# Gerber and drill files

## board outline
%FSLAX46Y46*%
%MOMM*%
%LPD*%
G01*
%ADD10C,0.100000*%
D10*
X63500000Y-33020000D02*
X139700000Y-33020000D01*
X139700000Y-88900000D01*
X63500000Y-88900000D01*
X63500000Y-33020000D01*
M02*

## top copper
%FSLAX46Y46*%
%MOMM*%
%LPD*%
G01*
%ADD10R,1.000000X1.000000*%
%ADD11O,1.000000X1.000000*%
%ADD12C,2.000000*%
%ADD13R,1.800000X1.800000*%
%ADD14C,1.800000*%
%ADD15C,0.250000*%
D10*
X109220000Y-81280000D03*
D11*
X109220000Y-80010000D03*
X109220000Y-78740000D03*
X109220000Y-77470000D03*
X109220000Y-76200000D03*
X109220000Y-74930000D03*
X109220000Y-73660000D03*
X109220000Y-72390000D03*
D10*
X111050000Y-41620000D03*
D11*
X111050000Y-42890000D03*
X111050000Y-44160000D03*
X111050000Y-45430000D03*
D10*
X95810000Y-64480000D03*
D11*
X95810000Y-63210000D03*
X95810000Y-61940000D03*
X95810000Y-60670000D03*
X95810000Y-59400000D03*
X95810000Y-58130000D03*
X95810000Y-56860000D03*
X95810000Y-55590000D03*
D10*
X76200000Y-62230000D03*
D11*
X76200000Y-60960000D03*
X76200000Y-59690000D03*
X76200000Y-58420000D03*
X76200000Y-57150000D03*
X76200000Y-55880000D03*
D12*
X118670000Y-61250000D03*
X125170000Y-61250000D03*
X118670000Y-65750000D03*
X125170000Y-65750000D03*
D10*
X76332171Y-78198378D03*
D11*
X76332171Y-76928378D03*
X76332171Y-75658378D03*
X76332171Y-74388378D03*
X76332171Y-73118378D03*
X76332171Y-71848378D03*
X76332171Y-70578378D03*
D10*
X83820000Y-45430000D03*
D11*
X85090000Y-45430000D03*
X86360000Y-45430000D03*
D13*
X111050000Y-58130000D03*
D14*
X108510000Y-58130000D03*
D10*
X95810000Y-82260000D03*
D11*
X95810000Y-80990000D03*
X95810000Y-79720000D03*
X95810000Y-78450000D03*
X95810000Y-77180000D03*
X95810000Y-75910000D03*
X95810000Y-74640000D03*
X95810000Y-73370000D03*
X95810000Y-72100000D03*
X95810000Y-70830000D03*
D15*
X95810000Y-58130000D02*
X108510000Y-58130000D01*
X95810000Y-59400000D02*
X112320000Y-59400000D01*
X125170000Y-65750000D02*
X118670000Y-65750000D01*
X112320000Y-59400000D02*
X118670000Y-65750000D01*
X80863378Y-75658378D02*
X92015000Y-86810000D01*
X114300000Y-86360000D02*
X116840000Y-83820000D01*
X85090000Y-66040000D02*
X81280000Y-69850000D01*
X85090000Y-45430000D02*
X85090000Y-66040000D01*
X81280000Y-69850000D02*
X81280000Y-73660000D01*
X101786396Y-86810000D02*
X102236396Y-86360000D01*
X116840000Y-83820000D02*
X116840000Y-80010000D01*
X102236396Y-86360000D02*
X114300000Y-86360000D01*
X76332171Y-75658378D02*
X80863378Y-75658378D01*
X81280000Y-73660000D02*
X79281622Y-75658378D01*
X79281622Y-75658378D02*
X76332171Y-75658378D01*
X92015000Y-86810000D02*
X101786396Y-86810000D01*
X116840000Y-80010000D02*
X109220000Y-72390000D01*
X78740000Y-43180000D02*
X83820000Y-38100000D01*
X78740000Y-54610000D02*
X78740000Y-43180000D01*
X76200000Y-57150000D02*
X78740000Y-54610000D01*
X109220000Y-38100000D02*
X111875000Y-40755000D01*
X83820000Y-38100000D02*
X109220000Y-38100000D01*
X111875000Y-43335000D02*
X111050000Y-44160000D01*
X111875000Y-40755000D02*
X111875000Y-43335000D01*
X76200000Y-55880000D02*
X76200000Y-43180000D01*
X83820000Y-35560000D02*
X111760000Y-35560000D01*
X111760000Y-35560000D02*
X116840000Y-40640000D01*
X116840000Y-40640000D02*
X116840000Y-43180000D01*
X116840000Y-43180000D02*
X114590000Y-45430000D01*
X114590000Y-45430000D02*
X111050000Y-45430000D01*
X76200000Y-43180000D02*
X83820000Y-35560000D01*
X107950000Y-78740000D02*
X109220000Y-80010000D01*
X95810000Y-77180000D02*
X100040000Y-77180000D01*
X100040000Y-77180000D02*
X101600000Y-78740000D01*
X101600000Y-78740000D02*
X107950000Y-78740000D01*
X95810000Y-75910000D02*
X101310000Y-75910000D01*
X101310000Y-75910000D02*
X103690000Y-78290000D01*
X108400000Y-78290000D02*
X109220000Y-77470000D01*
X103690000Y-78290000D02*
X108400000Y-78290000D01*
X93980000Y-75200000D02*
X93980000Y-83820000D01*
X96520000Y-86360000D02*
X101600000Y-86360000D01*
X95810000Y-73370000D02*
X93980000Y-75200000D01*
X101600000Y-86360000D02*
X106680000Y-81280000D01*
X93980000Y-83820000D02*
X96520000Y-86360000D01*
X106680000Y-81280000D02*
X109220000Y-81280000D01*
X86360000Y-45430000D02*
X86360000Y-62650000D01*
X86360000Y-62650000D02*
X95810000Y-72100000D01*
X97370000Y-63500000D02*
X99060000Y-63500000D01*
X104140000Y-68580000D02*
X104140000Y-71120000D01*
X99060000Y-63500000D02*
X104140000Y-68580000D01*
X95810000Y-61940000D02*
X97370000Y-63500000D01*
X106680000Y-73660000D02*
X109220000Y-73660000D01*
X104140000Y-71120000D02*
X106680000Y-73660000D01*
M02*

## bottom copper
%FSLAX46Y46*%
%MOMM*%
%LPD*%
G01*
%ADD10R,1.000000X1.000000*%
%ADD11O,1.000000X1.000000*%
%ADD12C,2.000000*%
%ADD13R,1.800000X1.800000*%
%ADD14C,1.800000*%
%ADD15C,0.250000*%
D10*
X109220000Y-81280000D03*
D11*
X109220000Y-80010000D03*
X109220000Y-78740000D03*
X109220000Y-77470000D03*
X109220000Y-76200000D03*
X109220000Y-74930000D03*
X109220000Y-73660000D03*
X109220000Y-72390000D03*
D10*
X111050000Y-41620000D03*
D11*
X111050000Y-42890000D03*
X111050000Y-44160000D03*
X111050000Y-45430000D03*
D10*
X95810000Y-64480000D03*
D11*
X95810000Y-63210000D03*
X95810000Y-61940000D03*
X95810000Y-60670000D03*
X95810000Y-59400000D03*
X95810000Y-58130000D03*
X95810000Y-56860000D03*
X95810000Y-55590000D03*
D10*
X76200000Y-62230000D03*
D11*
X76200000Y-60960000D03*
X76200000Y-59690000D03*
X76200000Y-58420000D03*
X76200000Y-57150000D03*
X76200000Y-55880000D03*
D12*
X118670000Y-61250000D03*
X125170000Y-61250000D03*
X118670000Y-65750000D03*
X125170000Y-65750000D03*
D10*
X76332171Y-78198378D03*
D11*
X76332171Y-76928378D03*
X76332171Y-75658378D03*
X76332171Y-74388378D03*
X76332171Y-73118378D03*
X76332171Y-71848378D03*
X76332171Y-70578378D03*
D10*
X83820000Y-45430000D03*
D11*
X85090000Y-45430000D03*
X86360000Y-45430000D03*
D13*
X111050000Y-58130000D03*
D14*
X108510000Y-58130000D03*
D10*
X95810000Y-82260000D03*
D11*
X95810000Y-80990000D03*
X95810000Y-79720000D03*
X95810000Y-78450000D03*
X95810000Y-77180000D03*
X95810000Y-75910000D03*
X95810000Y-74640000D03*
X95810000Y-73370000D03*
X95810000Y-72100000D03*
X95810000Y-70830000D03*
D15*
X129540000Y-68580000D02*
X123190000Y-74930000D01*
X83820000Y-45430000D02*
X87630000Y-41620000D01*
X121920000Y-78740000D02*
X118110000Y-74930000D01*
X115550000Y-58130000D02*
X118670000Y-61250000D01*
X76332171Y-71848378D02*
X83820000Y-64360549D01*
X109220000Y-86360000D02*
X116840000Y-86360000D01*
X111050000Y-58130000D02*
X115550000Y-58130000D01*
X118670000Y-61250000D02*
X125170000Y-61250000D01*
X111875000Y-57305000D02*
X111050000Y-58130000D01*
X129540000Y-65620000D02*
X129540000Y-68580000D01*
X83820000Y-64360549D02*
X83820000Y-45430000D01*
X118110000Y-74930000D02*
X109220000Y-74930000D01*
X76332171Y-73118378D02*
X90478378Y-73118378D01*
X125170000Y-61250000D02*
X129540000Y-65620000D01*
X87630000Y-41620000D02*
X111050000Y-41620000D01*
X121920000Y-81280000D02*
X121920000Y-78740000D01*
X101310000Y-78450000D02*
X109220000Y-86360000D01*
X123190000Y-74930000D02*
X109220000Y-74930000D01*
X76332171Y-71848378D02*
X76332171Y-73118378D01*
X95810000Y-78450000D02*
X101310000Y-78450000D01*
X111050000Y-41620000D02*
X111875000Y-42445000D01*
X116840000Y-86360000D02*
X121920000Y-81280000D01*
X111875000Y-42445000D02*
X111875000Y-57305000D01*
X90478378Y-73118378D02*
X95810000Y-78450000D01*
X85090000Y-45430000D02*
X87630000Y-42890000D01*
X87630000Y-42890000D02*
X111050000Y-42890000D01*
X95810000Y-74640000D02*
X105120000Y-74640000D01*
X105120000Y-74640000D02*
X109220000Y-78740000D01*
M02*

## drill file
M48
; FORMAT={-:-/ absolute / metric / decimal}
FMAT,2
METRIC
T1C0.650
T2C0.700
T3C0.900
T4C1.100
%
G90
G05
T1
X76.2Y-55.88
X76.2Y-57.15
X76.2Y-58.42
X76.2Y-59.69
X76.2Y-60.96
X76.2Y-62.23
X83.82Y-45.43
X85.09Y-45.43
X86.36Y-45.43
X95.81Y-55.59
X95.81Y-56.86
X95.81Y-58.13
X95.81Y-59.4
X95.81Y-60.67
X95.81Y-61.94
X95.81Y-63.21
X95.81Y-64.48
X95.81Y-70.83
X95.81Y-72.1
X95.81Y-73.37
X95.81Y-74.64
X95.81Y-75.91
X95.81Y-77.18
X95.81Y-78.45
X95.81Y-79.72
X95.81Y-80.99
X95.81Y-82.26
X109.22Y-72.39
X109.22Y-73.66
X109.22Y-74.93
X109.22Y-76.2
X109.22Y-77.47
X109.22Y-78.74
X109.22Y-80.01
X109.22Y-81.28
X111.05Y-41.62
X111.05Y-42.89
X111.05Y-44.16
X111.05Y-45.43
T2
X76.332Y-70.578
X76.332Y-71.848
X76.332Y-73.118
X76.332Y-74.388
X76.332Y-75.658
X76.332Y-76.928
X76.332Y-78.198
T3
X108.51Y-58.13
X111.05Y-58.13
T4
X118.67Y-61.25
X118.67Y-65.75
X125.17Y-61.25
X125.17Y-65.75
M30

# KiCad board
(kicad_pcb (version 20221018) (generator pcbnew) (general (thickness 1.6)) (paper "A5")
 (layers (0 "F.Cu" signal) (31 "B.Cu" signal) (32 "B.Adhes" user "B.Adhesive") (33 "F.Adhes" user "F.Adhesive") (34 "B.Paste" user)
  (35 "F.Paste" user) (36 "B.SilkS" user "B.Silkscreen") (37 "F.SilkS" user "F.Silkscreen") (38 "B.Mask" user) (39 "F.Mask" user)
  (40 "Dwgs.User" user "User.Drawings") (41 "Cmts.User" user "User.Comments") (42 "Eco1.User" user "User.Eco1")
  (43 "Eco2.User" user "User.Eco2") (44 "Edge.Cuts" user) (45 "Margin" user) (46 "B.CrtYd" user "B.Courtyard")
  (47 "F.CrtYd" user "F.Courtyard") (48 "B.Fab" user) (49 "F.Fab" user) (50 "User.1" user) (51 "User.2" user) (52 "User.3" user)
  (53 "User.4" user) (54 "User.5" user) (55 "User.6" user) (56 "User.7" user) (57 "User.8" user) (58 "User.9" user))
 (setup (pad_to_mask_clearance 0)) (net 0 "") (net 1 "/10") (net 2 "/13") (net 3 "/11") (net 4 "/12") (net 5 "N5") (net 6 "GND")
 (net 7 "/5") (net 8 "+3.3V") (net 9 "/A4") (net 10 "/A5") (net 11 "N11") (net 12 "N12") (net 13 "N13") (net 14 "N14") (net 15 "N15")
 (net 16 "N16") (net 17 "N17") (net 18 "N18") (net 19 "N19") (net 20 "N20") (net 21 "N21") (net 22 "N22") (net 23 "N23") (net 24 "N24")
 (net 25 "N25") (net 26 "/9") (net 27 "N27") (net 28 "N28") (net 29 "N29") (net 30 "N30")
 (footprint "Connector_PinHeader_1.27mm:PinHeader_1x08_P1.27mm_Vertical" (layer "F.Cu") (at 109.22 81.28 180)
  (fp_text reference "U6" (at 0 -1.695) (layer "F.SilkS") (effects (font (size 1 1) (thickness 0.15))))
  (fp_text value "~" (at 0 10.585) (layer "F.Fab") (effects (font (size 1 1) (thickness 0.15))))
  (pad "1" thru_hole rect (at 0 0 180) (size 1 1) (drill 0.65) (layers "*.Cu" "*.Mask") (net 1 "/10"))
  (pad "2" thru_hole oval (at 0 1.27 180) (size 1 1) (drill 0.65) (layers "*.Cu" "*.Mask") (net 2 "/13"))
  (pad "3" thru_hole oval (at 0 2.54 180) (size 1 1) (drill 0.65) (layers "*.Cu" "*.Mask") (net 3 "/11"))
  (pad "4" thru_hole oval (at 0 3.81 180) (size 1 1) (drill 0.65) (layers "*.Cu" "*.Mask") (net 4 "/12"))
  (pad "5" thru_hole oval (at 0 5.08 180) (size 1 1) (drill 0.65) (layers "*.Cu" "*.Mask") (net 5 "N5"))
  (pad "6" thru_hole oval (at 0 6.35 180) (size 1 1) (drill 0.65) (layers "*.Cu" "*.Mask") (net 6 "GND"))
  (pad "7" thru_hole oval (at 0 7.62 180) (size 1 1) (drill 0.65) (layers "*.Cu" "*.Mask") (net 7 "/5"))
  (pad "8" thru_hole oval (at 0 8.89 180) (size 1 1) (drill 0.65) (layers "*.Cu" "*.Mask") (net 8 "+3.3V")))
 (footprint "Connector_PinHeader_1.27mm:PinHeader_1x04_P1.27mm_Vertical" (layer "F.Cu") (at 111.05 41.62)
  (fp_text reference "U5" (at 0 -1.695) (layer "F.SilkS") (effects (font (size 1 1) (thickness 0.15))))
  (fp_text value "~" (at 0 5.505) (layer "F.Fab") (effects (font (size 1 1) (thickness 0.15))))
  (pad "1" thru_hole rect (at 0 0) (size 1 1) (drill 0.65) (layers "*.Cu" "*.Mask") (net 6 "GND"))
  (pad "2" thru_hole oval (at 0 1.27) (size 1 1) (drill 0.65) (layers "*.Cu" "*.Mask") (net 8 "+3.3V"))
  (pad "3" thru_hole oval (at 0 2.54) (size 1 1) (drill 0.65) (layers "*.Cu" "*.Mask") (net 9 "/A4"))
  (pad "4" thru_hole oval (at 0 3.81) (size 1 1) (drill 0.65) (layers "*.Cu" "*.Mask") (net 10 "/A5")))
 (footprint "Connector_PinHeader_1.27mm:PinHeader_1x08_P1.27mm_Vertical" (layer "F.Cu") (at 95.81 64.48 180)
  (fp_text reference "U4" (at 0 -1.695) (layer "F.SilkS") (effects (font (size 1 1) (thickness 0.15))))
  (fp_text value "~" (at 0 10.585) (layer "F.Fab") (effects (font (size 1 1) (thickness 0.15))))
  (pad "1" thru_hole rect (at 0 0 180) (size 1 1) (drill 0.65) (layers "*.Cu" "*.Mask") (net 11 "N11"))
  (pad "2" thru_hole oval (at 0 1.27 180) (size 1 1) (drill 0.65) (layers "*.Cu" "*.Mask") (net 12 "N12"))
  (pad "3" thru_hole oval (at 0 2.54 180) (size 1 1) (drill 0.65) (layers "*.Cu" "*.Mask") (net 7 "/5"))
  (pad "4" thru_hole oval (at 0 3.81 180) (size 1 1) (drill 0.65) (layers "*.Cu" "*.Mask") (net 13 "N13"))
  (pad "5" thru_hole oval (at 0 5.08 180) (size 1 1) (drill 0.65) (layers "*.Cu" "*.Mask") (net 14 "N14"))
  (pad "6" thru_hole oval (at 0 6.35 180) (size 1 1) (drill 0.65) (layers "*.Cu" "*.Mask") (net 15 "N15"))
  (pad "7" thru_hole oval (at 0 7.62 180) (size 1 1) (drill 0.65) (layers "*.Cu" "*.Mask") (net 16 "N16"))
  (pad "8" thru_hole oval (at 0 8.89 180) (size 1 1) (drill 0.65) (layers "*.Cu" "*.Mask") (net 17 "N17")))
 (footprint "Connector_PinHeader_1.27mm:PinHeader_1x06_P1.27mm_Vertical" (layer "F.Cu") (at 76.2 62.23 180)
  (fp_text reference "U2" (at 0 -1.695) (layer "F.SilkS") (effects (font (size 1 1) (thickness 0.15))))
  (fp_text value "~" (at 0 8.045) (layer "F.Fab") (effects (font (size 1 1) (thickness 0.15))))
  (pad "1" thru_hole rect (at 0 0 180) (size 1 1) (drill 0.65) (layers "*.Cu" "*.Mask") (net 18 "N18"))
  (pad "2" thru_hole oval (at 0 1.27 180) (size 1 1) (drill 0.65) (layers "*.Cu" "*.Mask") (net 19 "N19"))
  (pad "3" thru_hole oval (at 0 2.54 180) (size 1 1) (drill 0.65) (layers "*.Cu" "*.Mask") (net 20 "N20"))
  (pad "4" thru_hole oval (at 0 3.81 180) (size 1 1) (drill 0.65) (layers "*.Cu" "*.Mask") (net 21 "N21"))
  (pad "5" thru_hole oval (at 0 5.08 180) (size 1 1) (drill 0.65) (layers "*.Cu" "*.Mask") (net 9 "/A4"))
  (pad "6" thru_hole oval (at 0 6.35 180) (size 1 1) (drill 0.65) (layers "*.Cu" "*.Mask") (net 10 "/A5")))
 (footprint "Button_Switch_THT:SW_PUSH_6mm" (layer "F.Cu") (at 118.67 61.25)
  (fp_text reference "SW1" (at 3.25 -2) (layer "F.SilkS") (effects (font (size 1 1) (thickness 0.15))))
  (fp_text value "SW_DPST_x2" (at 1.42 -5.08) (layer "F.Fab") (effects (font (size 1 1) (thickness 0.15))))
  (pad "1" thru_hole circle (at 0 0 90) (size 2 2) (drill 1.1) (layers "*.Cu" "*.Mask") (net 6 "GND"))
  (pad "1" thru_hole circle (at 6.5 0 90) (size 2 2) (drill 1.1) (layers "*.Cu" "*.Mask") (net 6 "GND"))
  (pad "2" thru_hole circle (at 0 4.5 90) (size 2 2) (drill 1.1) (layers "*.Cu" "*.Mask") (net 14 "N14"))
  (pad "2" thru_hole circle (at 6.5 4.5 90) (size 2 2) (drill 1.1) (layers "*.Cu" "*.Mask") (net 14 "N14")))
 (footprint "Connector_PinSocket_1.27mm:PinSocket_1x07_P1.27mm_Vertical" (layer "F.Cu") (at 76.332171 78.198378 180)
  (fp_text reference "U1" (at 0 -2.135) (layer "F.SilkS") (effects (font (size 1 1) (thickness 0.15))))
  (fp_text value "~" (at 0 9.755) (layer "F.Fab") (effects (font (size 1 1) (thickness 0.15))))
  (pad "1" thru_hole rect (at 0 0 180) (size 1 1) (drill 0.7) (layers "*.Cu" "*.Mask") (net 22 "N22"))
  (pad "2" thru_hole oval (at 0 1.27 180) (size 1 1) (drill 0.7) (layers "*.Cu" "*.Mask") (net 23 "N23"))
  (pad "3" thru_hole oval (at 0 2.54 180) (size 1 1) (drill 0.7) (layers "*.Cu" "*.Mask") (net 8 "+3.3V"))
  (pad "4" thru_hole oval (at 0 3.81 180) (size 1 1) (drill 0.7) (layers "*.Cu" "*.Mask") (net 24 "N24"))
  (pad "5" thru_hole oval (at 0 5.08 180) (size 1 1) (drill 0.7) (layers "*.Cu" "*.Mask") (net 6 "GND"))
  (pad "6" thru_hole oval (at 0 6.35 180) (size 1 1) (drill 0.7) (layers "*.Cu" "*.Mask") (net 6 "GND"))
  (pad "7" thru_hole oval (at 0 7.62 180) (size 1 1) (drill 0.7) (layers "*.Cu" "*.Mask") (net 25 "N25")))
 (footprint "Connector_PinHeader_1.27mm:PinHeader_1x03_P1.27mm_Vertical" (layer "F.Cu") (at 83.82 45.43 90)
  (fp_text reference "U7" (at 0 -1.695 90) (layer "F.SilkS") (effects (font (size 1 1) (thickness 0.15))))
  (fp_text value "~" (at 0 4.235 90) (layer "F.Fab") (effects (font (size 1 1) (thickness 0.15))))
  (pad "1" thru_hole rect (at 0 0 90) (size 1 1) (drill 0.65) (layers "*.Cu" "*.Mask") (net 6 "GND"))
  (pad "2" thru_hole oval (at 0 1.27 90) (size 1 1) (drill 0.65) (layers "*.Cu" "*.Mask") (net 8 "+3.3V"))
  (pad "3" thru_hole oval (at 0 2.54 90) (size 1 1) (drill 0.65) (layers "*.Cu" "*.Mask") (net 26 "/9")))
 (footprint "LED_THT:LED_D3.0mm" (layer "F.Cu") (at 111.05 58.13 180)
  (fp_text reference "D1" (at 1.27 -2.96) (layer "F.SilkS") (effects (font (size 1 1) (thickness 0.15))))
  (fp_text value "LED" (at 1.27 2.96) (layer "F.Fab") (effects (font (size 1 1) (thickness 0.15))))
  (pad "1" thru_hole rect (at 0 0 180) (size 1.8 1.8) (drill 0.9) (layers "*.Cu" "*.Mask") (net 6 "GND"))
  (pad "2" thru_hole circle (at 2.54 0 180) (size 1.8 1.8) (drill 0.9) (layers "*.Cu" "*.Mask") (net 15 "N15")))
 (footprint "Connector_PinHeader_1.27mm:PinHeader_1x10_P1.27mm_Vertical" (layer "F.Cu") (at 95.81 82.26 180)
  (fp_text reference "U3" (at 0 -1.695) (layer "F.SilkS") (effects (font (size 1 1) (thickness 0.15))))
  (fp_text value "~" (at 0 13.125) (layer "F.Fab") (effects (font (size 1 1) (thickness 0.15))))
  (pad "1" thru_hole rect (at 0 0 180) (size 1 1) (drill 0.65) (layers "*.Cu" "*.Mask") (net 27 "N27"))
  (pad "2" thru_hole oval (at 0 1.27 180) (size 1 1) (drill 0.65) (layers "*.Cu" "*.Mask") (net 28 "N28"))
  (pad "3" thru_hole oval (at 0 2.54 180) (size 1 1) (drill 0.65) (layers "*.Cu" "*.Mask") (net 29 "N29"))
  (pad "4" thru_hole oval (at 0 3.81 180) (size 1 1) (drill 0.65) (layers "*.Cu" "*.Mask") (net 6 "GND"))
  (pad "5" thru_hole oval (at 0 5.08 180) (size 1 1) (drill 0.65) (layers "*.Cu" "*.Mask") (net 2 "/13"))
  (pad "6" thru_hole oval (at 0 6.35 180) (size 1 1) (drill 0.65) (layers "*.Cu" "*.Mask") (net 4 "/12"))
  (pad "7" thru_hole oval (at 0 7.62 180) (size 1 1) (drill 0.65) (layers "*.Cu" "*.Mask") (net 3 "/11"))
  (pad "8" thru_hole oval (at 0 8.89 180) (size 1 1) (drill 0.65) (layers "*.Cu" "*.Mask") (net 1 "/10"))
  (pad "9" thru_hole oval (at 0 10.16 180) (size 1 1) (drill 0.65) (layers "*.Cu" "*.Mask") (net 26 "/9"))
  (pad "10" thru_hole oval (at 0 11.43 180) (size 1 1) (drill 0.65) (layers "*.Cu" "*.Mask") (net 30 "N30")))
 (gr_rect (start 63.5 33.02) (end 139.7 88.9) (stroke (width 0.1) (type default)) (fill none) (layer "Edge.Cuts"))
 (segment (start 129.54 68.58) (end 123.19 74.93) (width 0.25) (layer "B.Cu") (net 6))
 (segment (start 83.82 45.43) (end 87.63 41.62) (width 0.25) (layer "B.Cu") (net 6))
 (segment (start 121.92 78.74) (end 118.11 74.93) (width 0.25) (layer "B.Cu") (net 6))
 (segment (start 115.55 58.13) (end 118.67 61.25) (width 0.25) (layer "B.Cu") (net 6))
 (segment (start 76.332171 71.848378) (end 83.82 64.360549) (width 0.25) (layer "B.Cu") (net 6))
 (segment (start 109.22 86.36) (end 116.84 86.36) (width 0.25) (layer "B.Cu") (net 6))
 (segment (start 111.05 58.13) (end 115.55 58.13) (width 0.25) (layer "B.Cu") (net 6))
 (segment (start 118.67 61.25) (end 125.17 61.25) (width 0.25) (layer "B.Cu") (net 6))
 (segment (start 111.875 57.305) (end 111.05 58.13) (width 0.25) (layer "B.Cu") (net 6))
 (segment (start 129.54 65.62) (end 129.54 68.58) (width 0.25) (layer "B.Cu") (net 6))
 (segment (start 83.82 64.360549) (end 83.82 45.43) (width 0.25) (layer "B.Cu") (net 6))
 (segment (start 118.11 74.93) (end 109.22 74.93) (width 0.25) (layer "B.Cu") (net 6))
 (segment (start 76.332171 73.118378) (end 90.478378 73.118378) (width 0.25) (layer "B.Cu") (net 6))
 (segment (start 125.17 61.25) (end 129.54 65.62) (width 0.25) (layer "B.Cu") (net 6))
 (segment (start 87.63 41.62) (end 111.05 41.62) (width 0.25) (layer "B.Cu") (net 6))
 (segment (start 121.92 81.28) (end 121.92 78.74) (width 0.25) (layer "B.Cu") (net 6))
 (segment (start 101.31 78.45) (end 109.22 86.36) (width 0.25) (layer "B.Cu") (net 6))
 (segment (start 123.19 74.93) (end 109.22 74.93) (width 0.25) (layer "B.Cu") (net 6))
 (segment (start 76.332171 71.848378) (end 76.332171 73.118378) (width 0.25) (layer "B.Cu") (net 6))
 (segment (start 95.81 78.45) (end 101.31 78.45) (width 0.25) (layer "B.Cu") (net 6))
 (segment (start 111.05 41.62) (end 111.875 42.445) (width 0.25) (layer "B.Cu") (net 6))
 (segment (start 116.84 86.36) (end 121.92 81.28) (width 0.25) (layer "B.Cu") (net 6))
 (segment (start 111.875 42.445) (end 111.875 57.305) (width 0.25) (layer "B.Cu") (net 6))
 (segment (start 90.478378 73.118378) (end 95.81 78.45) (width 0.25) (layer "B.Cu") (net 6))
 (segment (start 95.81 58.13) (end 108.51 58.13) (width 0.25) (layer "F.Cu") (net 15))
 (segment (start 95.81 59.4) (end 112.32 59.4) (width 0.25) (layer "F.Cu") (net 14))
 (segment (start 125.17 65.75) (end 118.67 65.75) (width 0.25) (layer "F.Cu") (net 14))
 (segment (start 112.32 59.4) (end 118.67 65.75) (width 0.25) (layer "F.Cu") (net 14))
 (segment (start 80.863378 75.658378) (end 92.015 86.81) (width 0.25) (layer "F.Cu") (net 8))
 (segment (start 114.3 86.36) (end 116.84 83.82) (width 0.25) (layer "F.Cu") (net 8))
 (segment (start 85.09 66.04) (end 81.28 69.85) (width 0.25) (layer "F.Cu") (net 8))
 (segment (start 85.09 45.43) (end 85.09 66.04) (width 0.25) (layer "F.Cu") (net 8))
 (segment (start 81.28 69.85) (end 81.28 73.66) (width 0.25) (layer "F.Cu") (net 8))
 (segment (start 101.786396 86.81) (end 102.236396 86.36) (width 0.25) (layer "F.Cu") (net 8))
 (segment (start 116.84 83.82) (end 116.84 80.01) (width 0.25) (layer "F.Cu") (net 8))
 (segment (start 102.236396 86.36) (end 114.3 86.36) (width 0.25) (layer "F.Cu") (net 8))
 (segment (start 76.332171 75.658378) (end 80.863378 75.658378) (width 0.25) (layer "F.Cu") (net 8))
 (segment (start 81.28 73.66) (end 79.281622 75.658378) (width 0.25) (layer "F.Cu") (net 8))
 (segment (start 79.281622 75.658378) (end 76.332171 75.658378) (width 0.25) (layer "F.Cu") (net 8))
 (segment (start 92.015 86.81) (end 101.786396 86.81) (width 0.25) (layer "F.Cu") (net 8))
 (segment (start 116.84 80.01) (end 109.22 72.39) (width 0.25) (layer "F.Cu") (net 8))
 (segment (start 85.09 45.43) (end 87.63 42.89) (width 0.25) (layer "B.Cu") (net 8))
 (segment (start 87.63 42.89) (end 111.05 42.89) (width 0.25) (layer "B.Cu") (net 8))
 (segment (start 78.74 43.18) (end 83.82 38.1) (width 0.25) (layer "F.Cu") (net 9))
 (segment (start 78.74 54.61) (end 78.74 43.18) (width 0.25) (layer "F.Cu") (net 9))
 (segment (start 76.2 57.15) (end 78.74 54.61) (width 0.25) (layer "F.Cu") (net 9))
 (segment (start 109.22 38.1) (end 111.875 40.755) (width 0.25) (layer "F.Cu") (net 9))
 (segment (start 83.82 38.1) (end 109.22 38.1) (width 0.25) (layer "F.Cu") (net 9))
 (segment (start 111.875 43.335) (end 111.05 44.16) (width 0.25) (layer "F.Cu") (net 9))
 (segment (start 111.875 40.755) (end 111.875 43.335) (width 0.25) (layer "F.Cu") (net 9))
 (segment (start 76.2 55.88) (end 76.2 43.18) (width 0.25) (layer "F.Cu") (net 10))
 (segment (start 83.82 35.56) (end 111.76 35.56) (width 0.25) (layer "F.Cu") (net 10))
 (segment (start 111.76 35.56) (end 116.84 40.64) (width 0.25) (layer "F.Cu") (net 10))
 (segment (start 116.84 40.64) (end 116.84 43.18) (width 0.25) (layer "F.Cu") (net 10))
 (segment (start 116.84 43.18) (end 114.59 45.43) (width 0.25) (layer "F.Cu") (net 10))
 (segment (start 114.59 45.43) (end 111.05 45.43) (width 0.25) (layer "F.Cu") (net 10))
 (segment (start 76.2 43.18) (end 83.82 35.56) (width 0.25) (layer "F.Cu") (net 10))
 (segment (start 107.95 78.74) (end 109.22 80.01) (width 0.25) (layer "F.Cu") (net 2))
 (segment (start 95.81 77.18) (end 100.04 77.18) (width 0.25) (layer "F.Cu") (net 2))
 (segment (start 100.04 77.18) (end 101.6 78.74) (width 0.25) (layer "F.Cu") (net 2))
 (segment (start 101.6 78.74) (end 107.95 78.74) (width 0.25) (layer "F.Cu") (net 2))
 (segment (start 95.81 75.91) (end 101.31 75.91) (width 0.25) (layer "F.Cu") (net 4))
 (segment (start 101.31 75.91) (end 103.69 78.29) (width 0.25) (layer "F.Cu") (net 4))
 (segment (start 108.4 78.29) (end 109.22 77.47) (width 0.25) (layer "F.Cu") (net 4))
 (segment (start 103.69 78.29) (end 108.4 78.29) (width 0.25) (layer "F.Cu") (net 4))
 (segment (start 95.81 74.64) (end 105.12 74.64) (width 0.25) (layer "B.Cu") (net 3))
 (segment (start 105.12 74.64) (end 109.22 78.74) (width 0.25) (layer "B.Cu") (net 3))
 (segment (start 93.98 75.2) (end 93.98 83.82) (width 0.25) (layer "F.Cu") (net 1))
 (segment (start 96.52 86.36) (end 101.6 86.36) (width 0.25) (layer "F.Cu") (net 1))
 (segment (start 95.81 73.37) (end 93.98 75.2) (width 0.25) (layer "F.Cu") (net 1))
 (segment (start 101.6 86.36) (end 106.68 81.28) (width 0.25) (layer "F.Cu") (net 1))
 (segment (start 93.98 83.82) (end 96.52 86.36) (width 0.25) (layer "F.Cu") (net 1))
 (segment (start 106.68 81.28) (end 109.22 81.28) (width 0.25) (layer "F.Cu") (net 1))
 (segment (start 86.36 45.43) (end 86.36 62.65) (width 0.25) (layer "F.Cu") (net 26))
 (segment (start 86.36 62.65) (end 95.81 72.1) (width 0.25) (layer "F.Cu") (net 26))
 (segment (start 97.37 63.5) (end 99.06 63.5) (width 0.25) (layer "F.Cu") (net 7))
 (segment (start 104.14 68.58) (end 104.14 71.12) (width 0.25) (layer "F.Cu") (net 7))
 (segment (start 99.06 63.5) (end 104.14 68.58) (width 0.25) (layer "F.Cu") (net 7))
 (segment (start 95.81 61.94) (end 97.37 63.5) (width 0.25) (layer "F.Cu") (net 7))
 (segment (start 106.68 73.66) (end 109.22 73.66) (width 0.25) (layer "F.Cu") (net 7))
 (segment (start 104.14 71.12) (end 106.68 73.66) (width 0.25) (layer "F.Cu") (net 7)))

